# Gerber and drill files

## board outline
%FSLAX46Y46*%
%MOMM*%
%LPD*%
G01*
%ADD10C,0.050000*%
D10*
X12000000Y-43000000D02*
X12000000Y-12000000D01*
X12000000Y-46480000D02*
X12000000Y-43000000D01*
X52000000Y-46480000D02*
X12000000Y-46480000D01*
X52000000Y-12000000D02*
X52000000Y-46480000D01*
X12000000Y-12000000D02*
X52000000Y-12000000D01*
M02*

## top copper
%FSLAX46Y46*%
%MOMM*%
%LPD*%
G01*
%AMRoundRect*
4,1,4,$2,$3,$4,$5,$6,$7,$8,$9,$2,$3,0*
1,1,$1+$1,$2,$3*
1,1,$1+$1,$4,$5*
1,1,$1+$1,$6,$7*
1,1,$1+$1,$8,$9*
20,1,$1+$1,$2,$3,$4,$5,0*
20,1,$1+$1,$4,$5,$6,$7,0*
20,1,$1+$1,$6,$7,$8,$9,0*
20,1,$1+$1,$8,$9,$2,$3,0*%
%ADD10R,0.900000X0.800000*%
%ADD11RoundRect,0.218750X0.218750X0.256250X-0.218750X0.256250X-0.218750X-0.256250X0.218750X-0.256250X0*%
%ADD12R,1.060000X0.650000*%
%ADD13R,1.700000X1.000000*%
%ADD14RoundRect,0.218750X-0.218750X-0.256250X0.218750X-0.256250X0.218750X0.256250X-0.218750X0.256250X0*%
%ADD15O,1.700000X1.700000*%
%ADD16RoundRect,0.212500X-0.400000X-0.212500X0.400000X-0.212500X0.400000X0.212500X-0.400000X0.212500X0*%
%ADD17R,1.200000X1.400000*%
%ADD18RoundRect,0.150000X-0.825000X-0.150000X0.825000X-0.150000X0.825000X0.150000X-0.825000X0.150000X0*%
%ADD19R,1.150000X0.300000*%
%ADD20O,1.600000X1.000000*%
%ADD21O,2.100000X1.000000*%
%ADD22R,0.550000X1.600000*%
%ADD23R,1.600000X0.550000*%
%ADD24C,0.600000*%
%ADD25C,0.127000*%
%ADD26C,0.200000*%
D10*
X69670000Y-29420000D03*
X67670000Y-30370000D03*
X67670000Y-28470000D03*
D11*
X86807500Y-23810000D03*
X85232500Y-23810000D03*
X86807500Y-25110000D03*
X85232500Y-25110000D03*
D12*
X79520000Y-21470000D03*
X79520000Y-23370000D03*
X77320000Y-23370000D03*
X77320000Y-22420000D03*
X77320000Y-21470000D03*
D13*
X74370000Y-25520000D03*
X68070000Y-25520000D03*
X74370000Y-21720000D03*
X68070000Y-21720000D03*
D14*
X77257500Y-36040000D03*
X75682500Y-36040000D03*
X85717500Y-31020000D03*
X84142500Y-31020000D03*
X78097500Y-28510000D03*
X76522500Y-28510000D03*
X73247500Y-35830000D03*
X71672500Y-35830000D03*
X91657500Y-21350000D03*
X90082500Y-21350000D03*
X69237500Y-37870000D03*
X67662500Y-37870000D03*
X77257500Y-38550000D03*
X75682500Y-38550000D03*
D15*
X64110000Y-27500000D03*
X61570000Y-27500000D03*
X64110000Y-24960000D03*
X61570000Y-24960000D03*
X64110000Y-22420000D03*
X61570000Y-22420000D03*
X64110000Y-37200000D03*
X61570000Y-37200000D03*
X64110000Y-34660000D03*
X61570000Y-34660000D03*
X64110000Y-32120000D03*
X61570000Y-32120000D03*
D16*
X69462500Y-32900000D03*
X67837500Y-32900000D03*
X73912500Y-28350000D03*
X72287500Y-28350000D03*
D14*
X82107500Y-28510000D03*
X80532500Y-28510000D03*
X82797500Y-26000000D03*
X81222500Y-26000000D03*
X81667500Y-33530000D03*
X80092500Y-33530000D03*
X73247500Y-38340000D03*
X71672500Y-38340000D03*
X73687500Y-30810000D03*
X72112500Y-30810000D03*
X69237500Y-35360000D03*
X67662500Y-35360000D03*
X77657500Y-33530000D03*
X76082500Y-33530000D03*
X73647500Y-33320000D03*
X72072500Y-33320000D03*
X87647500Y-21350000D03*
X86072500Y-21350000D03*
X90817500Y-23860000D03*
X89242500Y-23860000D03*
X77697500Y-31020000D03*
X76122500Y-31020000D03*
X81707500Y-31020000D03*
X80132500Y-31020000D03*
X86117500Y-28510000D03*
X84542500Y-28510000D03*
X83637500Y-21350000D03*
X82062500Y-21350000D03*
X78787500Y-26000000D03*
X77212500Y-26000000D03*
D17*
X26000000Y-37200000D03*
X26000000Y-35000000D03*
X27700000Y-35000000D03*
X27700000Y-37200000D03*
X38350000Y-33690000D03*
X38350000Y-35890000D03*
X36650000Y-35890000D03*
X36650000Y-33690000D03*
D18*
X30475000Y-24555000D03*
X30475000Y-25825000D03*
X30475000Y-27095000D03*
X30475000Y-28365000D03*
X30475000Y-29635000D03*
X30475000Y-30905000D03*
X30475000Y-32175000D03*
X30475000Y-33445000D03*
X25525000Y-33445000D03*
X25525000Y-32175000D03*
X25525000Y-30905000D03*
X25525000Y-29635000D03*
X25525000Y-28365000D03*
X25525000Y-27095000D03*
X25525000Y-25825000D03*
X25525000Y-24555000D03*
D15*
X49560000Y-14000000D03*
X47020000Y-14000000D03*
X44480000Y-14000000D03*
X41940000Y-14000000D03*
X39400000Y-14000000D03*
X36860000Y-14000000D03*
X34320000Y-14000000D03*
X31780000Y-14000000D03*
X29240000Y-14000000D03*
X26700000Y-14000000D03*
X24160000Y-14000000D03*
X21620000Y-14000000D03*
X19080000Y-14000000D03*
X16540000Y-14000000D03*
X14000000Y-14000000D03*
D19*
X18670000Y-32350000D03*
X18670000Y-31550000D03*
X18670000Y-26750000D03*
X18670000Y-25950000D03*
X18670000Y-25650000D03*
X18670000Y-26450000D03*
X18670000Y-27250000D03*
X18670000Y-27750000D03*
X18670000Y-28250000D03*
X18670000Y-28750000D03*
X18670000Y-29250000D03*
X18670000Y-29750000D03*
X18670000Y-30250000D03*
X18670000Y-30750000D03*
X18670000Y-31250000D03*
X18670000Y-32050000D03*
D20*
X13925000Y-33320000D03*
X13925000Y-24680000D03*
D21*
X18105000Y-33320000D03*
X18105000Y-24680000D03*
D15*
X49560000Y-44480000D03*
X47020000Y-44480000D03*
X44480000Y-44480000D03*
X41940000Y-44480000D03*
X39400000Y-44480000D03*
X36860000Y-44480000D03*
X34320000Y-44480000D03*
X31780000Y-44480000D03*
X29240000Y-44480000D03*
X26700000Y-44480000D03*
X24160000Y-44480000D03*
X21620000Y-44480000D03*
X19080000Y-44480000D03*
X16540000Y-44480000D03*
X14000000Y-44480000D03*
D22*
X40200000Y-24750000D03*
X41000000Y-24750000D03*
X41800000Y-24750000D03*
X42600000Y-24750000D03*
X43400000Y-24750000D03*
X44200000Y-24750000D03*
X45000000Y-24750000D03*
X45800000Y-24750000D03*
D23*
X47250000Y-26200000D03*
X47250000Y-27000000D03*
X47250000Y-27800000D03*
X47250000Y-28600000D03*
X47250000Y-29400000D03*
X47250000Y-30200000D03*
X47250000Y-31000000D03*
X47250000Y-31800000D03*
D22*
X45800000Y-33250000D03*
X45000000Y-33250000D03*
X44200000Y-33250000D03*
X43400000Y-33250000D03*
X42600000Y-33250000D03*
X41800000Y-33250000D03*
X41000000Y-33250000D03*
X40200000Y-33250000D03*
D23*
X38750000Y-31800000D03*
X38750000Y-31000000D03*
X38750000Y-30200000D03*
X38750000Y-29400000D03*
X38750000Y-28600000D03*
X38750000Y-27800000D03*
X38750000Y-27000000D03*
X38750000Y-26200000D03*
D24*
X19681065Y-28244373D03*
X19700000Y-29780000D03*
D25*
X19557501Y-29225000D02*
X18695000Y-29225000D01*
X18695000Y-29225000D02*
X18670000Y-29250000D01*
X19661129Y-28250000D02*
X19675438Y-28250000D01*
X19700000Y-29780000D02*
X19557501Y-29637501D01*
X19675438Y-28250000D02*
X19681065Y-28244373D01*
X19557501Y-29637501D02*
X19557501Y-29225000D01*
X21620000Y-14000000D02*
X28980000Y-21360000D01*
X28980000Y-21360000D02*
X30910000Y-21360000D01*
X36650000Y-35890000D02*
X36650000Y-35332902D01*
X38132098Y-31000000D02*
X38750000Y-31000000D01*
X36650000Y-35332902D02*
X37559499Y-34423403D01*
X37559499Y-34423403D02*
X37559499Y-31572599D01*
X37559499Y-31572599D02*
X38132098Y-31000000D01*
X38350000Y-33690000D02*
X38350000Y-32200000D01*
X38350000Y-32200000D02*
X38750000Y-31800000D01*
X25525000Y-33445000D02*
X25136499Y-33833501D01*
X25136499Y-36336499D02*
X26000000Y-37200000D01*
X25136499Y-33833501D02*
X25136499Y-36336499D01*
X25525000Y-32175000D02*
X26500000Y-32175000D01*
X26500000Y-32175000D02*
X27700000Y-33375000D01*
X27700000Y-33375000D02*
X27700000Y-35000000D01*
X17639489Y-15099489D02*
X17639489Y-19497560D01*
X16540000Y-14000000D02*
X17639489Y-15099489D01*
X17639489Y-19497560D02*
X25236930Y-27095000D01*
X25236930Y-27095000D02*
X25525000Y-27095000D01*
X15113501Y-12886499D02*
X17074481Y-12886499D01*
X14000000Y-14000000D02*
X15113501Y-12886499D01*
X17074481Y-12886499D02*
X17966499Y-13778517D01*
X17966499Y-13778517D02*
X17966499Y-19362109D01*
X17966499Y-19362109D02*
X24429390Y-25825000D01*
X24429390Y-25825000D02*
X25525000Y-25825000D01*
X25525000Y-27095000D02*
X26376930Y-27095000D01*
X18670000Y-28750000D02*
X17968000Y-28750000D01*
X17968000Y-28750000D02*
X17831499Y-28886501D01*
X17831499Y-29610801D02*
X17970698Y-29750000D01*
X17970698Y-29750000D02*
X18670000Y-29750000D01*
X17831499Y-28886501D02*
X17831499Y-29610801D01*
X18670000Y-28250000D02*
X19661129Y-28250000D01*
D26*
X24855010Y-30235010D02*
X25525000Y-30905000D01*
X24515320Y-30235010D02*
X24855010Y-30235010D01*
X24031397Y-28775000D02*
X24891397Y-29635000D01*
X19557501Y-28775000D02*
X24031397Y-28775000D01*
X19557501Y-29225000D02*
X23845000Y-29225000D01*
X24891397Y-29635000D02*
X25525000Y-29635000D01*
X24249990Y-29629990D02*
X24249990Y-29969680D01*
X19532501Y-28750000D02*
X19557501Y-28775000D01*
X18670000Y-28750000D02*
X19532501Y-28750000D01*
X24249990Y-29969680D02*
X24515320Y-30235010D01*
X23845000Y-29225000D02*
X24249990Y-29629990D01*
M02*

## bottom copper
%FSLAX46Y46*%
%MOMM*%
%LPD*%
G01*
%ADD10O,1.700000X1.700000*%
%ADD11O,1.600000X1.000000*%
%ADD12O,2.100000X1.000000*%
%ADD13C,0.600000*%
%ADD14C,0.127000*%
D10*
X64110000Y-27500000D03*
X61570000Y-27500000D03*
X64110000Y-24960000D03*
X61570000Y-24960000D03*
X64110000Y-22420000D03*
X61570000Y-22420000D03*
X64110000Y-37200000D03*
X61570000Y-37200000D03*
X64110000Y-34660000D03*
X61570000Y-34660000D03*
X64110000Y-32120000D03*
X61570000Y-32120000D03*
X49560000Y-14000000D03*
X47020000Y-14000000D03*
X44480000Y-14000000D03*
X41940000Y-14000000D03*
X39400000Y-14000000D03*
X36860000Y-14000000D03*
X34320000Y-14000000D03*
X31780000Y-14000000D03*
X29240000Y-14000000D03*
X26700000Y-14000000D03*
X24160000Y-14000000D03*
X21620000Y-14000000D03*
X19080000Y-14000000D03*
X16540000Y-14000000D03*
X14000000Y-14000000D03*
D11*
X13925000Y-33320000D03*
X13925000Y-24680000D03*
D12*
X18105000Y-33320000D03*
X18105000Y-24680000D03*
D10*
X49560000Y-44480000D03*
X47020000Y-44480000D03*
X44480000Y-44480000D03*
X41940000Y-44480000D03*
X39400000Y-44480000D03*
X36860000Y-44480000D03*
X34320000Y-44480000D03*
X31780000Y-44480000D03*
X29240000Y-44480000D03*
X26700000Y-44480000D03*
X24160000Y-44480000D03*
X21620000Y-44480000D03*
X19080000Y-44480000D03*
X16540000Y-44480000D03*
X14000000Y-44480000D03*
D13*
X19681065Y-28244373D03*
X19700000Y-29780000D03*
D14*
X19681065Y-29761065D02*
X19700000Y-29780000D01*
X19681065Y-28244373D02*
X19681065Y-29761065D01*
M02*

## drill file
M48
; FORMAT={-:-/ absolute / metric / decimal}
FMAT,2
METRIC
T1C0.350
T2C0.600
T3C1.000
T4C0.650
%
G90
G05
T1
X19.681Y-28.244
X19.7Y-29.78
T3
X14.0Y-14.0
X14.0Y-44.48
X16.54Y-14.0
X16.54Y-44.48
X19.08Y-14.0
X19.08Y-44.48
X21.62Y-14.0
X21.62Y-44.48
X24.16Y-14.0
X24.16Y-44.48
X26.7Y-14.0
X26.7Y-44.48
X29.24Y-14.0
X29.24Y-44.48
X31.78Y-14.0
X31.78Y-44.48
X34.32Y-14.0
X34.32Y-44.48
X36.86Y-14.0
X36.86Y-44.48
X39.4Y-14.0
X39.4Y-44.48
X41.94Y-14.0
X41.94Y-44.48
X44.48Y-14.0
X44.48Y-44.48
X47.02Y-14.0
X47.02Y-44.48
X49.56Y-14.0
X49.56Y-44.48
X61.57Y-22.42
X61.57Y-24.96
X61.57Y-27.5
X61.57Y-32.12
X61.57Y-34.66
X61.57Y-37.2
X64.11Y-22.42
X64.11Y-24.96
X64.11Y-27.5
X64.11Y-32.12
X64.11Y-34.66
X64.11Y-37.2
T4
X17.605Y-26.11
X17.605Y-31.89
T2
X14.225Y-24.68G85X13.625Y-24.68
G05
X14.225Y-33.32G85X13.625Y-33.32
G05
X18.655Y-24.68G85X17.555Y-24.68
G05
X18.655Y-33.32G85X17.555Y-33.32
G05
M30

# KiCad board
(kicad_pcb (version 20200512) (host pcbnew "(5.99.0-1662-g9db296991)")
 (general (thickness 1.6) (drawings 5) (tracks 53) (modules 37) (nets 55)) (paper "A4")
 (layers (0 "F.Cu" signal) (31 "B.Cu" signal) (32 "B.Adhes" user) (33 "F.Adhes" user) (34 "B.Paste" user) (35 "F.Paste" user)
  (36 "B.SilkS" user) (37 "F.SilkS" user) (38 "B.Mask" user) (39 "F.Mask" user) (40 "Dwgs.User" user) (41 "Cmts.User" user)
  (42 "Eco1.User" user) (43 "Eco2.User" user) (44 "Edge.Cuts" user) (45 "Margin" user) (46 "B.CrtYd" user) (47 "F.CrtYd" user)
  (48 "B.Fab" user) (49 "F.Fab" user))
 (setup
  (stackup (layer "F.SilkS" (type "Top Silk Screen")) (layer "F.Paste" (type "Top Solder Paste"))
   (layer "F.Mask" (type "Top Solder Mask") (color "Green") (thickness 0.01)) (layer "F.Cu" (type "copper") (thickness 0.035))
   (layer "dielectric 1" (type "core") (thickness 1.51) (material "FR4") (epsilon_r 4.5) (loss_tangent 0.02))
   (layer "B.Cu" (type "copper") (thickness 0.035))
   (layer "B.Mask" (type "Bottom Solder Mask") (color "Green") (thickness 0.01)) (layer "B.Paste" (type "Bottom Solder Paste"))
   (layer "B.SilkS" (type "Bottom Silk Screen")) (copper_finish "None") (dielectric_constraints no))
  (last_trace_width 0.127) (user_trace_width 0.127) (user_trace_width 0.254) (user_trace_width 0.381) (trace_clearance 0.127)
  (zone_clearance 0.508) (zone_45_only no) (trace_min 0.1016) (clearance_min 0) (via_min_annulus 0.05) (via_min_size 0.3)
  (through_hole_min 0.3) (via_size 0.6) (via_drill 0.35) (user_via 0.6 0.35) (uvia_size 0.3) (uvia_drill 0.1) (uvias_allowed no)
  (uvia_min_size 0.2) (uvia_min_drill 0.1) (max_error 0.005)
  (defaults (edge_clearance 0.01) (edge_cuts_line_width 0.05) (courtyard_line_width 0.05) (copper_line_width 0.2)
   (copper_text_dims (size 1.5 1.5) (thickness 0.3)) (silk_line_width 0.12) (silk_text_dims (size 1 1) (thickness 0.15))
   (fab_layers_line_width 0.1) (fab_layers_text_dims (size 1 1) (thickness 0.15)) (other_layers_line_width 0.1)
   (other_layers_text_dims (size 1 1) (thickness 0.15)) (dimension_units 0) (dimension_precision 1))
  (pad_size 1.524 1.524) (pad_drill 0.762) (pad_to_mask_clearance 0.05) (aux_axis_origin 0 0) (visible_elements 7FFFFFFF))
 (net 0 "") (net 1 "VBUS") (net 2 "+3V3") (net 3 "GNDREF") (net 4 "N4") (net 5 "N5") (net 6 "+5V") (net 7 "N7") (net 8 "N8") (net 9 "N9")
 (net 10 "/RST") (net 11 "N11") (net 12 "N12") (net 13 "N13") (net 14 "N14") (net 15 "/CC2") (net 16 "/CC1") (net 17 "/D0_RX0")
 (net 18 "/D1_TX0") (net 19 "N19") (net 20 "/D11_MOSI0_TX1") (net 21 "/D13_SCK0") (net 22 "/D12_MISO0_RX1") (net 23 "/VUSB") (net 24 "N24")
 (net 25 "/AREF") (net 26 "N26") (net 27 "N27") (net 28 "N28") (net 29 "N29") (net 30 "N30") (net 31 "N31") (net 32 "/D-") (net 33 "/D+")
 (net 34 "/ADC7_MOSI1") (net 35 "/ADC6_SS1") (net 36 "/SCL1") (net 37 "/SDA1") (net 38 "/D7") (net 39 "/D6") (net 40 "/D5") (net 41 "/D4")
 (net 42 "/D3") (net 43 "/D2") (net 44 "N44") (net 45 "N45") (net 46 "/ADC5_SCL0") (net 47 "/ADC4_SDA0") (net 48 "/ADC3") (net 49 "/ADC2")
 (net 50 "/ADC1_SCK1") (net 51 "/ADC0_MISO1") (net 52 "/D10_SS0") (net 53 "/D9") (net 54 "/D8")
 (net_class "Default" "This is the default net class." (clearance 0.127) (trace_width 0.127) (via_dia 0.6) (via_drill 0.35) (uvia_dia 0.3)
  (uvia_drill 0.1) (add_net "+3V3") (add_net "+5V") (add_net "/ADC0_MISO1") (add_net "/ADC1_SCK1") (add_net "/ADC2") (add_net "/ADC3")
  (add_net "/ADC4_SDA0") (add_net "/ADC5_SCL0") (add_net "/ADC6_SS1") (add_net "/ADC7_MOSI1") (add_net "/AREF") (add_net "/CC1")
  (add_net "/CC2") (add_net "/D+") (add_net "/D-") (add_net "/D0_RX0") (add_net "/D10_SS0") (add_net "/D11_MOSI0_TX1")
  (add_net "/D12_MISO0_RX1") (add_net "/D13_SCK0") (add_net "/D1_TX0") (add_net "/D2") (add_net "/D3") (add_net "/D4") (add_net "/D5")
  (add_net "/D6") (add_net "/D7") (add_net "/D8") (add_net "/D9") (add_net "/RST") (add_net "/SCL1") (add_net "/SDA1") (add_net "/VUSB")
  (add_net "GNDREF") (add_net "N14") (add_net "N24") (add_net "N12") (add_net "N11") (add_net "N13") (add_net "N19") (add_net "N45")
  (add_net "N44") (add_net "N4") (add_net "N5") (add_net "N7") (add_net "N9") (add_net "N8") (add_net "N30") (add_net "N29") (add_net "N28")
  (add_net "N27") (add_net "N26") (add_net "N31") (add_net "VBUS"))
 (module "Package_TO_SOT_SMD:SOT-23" (layer "F.Cu") (at 68.67 29.42)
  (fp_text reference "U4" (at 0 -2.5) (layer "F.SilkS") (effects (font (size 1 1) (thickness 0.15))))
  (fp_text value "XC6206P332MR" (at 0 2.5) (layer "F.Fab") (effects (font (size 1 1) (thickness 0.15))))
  (pad "3" smd rect (at 1 0) (size 0.9 0.8) (layers "F.Cu" "F.Paste" "F.Mask") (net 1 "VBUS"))
  (pad "2" smd rect (at -1 0.95) (size 0.9 0.8) (layers "F.Cu" "F.Paste" "F.Mask") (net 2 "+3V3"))
  (pad "1" smd rect (at -1 -0.95) (size 0.9 0.8) (layers "F.Cu" "F.Paste" "F.Mask") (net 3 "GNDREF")))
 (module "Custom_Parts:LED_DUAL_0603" (layer "F.Cu") (at 86.02 24.46)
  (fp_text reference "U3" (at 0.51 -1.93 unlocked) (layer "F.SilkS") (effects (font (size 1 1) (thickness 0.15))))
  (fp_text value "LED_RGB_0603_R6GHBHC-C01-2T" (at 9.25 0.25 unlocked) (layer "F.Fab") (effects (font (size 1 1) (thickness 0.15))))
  (pad "2" smd roundrect (at 0.7875 -0.65 180) (size 0.875 0.95) (layers "F.Cu" "F.Paste" "F.Mask") (roundrect_rratio 0.25) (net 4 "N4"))
  (pad "3" smd roundrect (at -0.7875 -0.65 180) (size 0.875 0.95) (layers "F.Cu" "F.Paste" "F.Mask") (roundrect_rratio 0.25) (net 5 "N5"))
  (pad "1" smd roundrect (at 0.7875 0.65 180) (size 0.875 0.95) (layers "F.Cu" "F.Paste" "F.Mask") (roundrect_rratio 0.25) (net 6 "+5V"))
  (pad "4" smd roundrect (at -0.7875 0.65 180) (size 0.875 0.95) (layers "F.Cu" "F.Paste" "F.Mask") (roundrect_rratio 0.25) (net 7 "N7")))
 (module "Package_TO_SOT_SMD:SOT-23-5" (layer "F.Cu") (at 78.42 22.42)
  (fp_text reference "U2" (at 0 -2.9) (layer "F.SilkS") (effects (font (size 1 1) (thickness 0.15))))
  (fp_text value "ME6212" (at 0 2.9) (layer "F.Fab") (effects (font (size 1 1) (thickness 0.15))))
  (pad "5" smd rect (at 1.1 -0.95) (size 1.06 0.65) (layers "F.Cu" "F.Paste" "F.Mask") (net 6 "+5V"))
  (pad "4" smd rect (at 1.1 0.95) (size 1.06 0.65) (layers "F.Cu" "F.Paste" "F.Mask") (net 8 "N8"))
  (pad "3" smd rect (at -1.1 0.95) (size 1.06 0.65) (layers "F.Cu" "F.Paste" "F.Mask") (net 1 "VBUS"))
  (pad "2" smd rect (at -1.1 0) (size 1.06 0.65) (layers "F.Cu" "F.Paste" "F.Mask") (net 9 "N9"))
  (pad "1" smd rect (at -1.1 -0.95) (size 1.06 0.65) (layers "F.Cu" "F.Paste" "F.Mask") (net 1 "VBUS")))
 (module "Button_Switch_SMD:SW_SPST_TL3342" (layer "F.Cu") (at 71.22 23.62)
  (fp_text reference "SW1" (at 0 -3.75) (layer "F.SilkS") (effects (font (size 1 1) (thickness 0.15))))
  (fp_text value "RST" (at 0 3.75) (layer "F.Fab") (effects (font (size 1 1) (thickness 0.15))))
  (pad "2" smd rect (at 3.15 1.9) (size 1.7 1) (layers "F.Cu" "F.Paste" "F.Mask") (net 3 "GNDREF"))
  (pad "2" smd rect (at -3.15 1.9) (size 1.7 1) (layers "F.Cu" "F.Paste" "F.Mask") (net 3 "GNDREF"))
  (pad "1" smd rect (at 3.15 -1.9) (size 1.7 1) (layers "F.Cu" "F.Paste" "F.Mask") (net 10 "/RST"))
  (pad "1" smd rect (at -3.15 -1.9) (size 1.7 1) (layers "F.Cu" "F.Paste" "F.Mask") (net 10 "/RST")))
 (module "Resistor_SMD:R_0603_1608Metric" (layer "F.Cu") (at 76.47 36.04)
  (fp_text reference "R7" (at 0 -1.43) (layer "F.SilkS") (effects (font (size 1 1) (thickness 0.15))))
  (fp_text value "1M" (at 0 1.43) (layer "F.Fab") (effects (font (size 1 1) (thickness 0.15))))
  (pad "2" smd roundrect (at 0.7875 0) (size 0.875 0.95) (layers "F.Cu" "F.Paste" "F.Mask") (roundrect_rratio 0.25) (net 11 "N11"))
  (pad "1" smd roundrect (at -0.7875 0) (size 0.875 0.95) (layers "F.Cu" "F.Paste" "F.Mask") (roundrect_rratio 0.25) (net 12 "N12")))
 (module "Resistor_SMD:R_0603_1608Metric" (layer "F.Cu") (at 84.93 31.02)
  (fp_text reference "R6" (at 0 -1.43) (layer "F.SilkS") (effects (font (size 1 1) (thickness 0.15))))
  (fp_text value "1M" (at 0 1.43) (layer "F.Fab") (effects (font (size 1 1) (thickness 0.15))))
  (pad "2" smd roundrect (at 0.7875 0) (size 0.875 0.95) (layers "F.Cu" "F.Paste" "F.Mask") (roundrect_rratio 0.25) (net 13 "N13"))
  (pad "1" smd roundrect (at -0.7875 0) (size 0.875 0.95) (layers "F.Cu" "F.Paste" "F.Mask") (roundrect_rratio 0.25) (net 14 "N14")))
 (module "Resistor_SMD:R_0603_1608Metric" (layer "F.Cu") (at 77.31 28.51)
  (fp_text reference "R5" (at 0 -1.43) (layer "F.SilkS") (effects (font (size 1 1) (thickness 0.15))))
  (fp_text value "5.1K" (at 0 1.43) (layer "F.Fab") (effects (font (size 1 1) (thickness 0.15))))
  (pad "2" smd roundrect (at 0.7875 0) (size 0.875 0.95) (layers "F.Cu" "F.Paste" "F.Mask") (roundrect_rratio 0.25) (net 3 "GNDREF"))
  (pad "1" smd roundrect (at -0.7875 0) (size 0.875 0.95) (layers "F.Cu" "F.Paste" "F.Mask") (roundrect_rratio 0.25) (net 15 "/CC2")))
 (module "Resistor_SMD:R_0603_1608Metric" (layer "F.Cu") (at 72.46 35.83)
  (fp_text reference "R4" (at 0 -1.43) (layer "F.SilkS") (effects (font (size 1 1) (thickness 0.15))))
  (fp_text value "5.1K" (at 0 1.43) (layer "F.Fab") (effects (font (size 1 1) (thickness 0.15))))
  (pad "2" smd roundrect (at 0.7875 0) (size 0.875 0.95) (layers "F.Cu" "F.Paste" "F.Mask") (roundrect_rratio 0.25) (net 3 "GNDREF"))
  (pad "1" smd roundrect (at -0.7875 0) (size 0.875 0.95) (layers "F.Cu" "F.Paste" "F.Mask") (roundrect_rratio 0.25) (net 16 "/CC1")))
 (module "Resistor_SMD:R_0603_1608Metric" (layer "F.Cu") (at 90.87 21.35)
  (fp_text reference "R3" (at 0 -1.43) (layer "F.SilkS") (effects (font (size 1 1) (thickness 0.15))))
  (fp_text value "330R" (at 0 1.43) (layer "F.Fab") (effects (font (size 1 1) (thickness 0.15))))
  (pad "2" smd roundrect (at 0.7875 0) (size 0.875 0.95) (layers "F.Cu" "F.Paste" "F.Mask") (roundrect_rratio 0.25) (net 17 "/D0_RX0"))
  (pad "1" smd roundrect (at -0.7875 0) (size 0.875 0.95) (layers "F.Cu" "F.Paste" "F.Mask") (roundrect_rratio 0.25) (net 7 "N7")))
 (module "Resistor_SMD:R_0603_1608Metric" (layer "F.Cu") (at 68.45 37.87)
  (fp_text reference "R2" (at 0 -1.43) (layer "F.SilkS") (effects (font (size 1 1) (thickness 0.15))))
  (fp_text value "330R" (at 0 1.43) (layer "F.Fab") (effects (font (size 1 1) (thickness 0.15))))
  (pad "2" smd roundrect (at 0.7875 0) (size 0.875 0.95) (layers "F.Cu" "F.Paste" "F.Mask") (roundrect_rratio 0.25) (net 3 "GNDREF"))
  (pad "1" smd roundrect (at -0.7875 0) (size 0.875 0.95) (layers "F.Cu" "F.Paste" "F.Mask") (roundrect_rratio 0.25) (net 5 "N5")))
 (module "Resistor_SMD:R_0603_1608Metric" (layer "F.Cu") (at 76.47 38.55)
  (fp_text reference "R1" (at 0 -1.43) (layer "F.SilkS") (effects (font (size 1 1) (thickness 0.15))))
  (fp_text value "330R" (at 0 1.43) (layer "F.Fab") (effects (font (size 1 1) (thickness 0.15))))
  (pad "2" smd roundrect (at 0.7875 0) (size 0.875 0.95) (layers "F.Cu" "F.Paste" "F.Mask") (roundrect_rratio 0.25) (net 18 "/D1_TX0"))
  (pad "1" smd roundrect (at -0.7875 0) (size 0.875 0.95) (layers "F.Cu" "F.Paste" "F.Mask") (roundrect_rratio 0.25) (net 4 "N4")))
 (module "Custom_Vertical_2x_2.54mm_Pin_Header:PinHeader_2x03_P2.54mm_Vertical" (layer "F.Cu") (at 61.57 22.42)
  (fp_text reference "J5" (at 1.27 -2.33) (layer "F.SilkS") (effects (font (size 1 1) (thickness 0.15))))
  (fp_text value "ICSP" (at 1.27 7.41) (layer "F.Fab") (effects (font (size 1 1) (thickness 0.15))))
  (pad "6" thru_hole oval (at 2.54 5.08) (size 1.7 1.7) (drill 1) (layers *.Cu *.Mask) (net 3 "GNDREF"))
  (pad "5" thru_hole oval (at 0 5.08) (size 1.7 1.7) (drill 1) (layers *.Cu *.Mask) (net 3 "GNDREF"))
  (pad "4" thru_hole oval (at 2.54 2.54) (size 1.7 1.7) (drill 1) (layers *.Cu *.Mask) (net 6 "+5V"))
  (pad "3" thru_hole oval (at 0 2.54) (size 1.7 1.7) (drill 1) (layers *.Cu *.Mask) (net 2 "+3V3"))
  (pad "2" thru_hole oval (at 2.54 0) (size 1.7 1.7) (drill 1) (layers *.Cu *.Mask) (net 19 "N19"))
  (pad "1" thru_hole oval (at 0 0) (size 1.7 1.7) (drill 1) (layers *.Cu *.Mask) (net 6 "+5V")))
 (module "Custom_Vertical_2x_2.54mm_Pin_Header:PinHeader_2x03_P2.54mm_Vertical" (layer "F.Cu") (at 61.57 32.12)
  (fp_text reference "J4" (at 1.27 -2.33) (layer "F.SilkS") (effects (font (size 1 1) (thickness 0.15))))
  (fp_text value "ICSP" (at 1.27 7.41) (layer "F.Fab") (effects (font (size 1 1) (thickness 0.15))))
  (pad "6" thru_hole oval (at 2.54 5.08) (size 1.7 1.7) (drill 1) (layers *.Cu *.Mask) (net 3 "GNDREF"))
  (pad "5" thru_hole oval (at 0 5.08) (size 1.7 1.7) (drill 1) (layers *.Cu *.Mask) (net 10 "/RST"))
  (pad "4" thru_hole oval (at 2.54 2.54) (size 1.7 1.7) (drill 1) (layers *.Cu *.Mask) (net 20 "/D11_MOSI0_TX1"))
  (pad "3" thru_hole oval (at 0 2.54) (size 1.7 1.7) (drill 1) (layers *.Cu *.Mask) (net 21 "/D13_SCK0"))
  (pad "2" thru_hole oval (at 2.54 0) (size 1.7 1.7) (drill 1) (layers *.Cu *.Mask) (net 6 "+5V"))
  (pad "1" thru_hole oval (at 0 0) (size 1.7 1.7) (drill 1) (layers *.Cu *.Mask) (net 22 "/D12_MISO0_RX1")))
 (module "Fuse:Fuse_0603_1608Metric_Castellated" (layer "F.Cu") (at 68.65 32.9)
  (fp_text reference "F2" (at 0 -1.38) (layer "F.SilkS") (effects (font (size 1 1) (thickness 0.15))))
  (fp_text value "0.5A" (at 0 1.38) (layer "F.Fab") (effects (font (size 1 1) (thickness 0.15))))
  (pad "2" smd roundrect (at 0.8125 0) (size 1.225 0.85) (layers "F.Cu" "F.Paste" "F.Mask") (roundrect_rratio 0.25) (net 1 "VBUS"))
  (pad "1" smd roundrect (at -0.8125 0) (size 1.225 0.85) (layers "F.Cu" "F.Paste" "F.Mask") (roundrect_rratio 0.25) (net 19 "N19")))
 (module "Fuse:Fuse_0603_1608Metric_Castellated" (layer "F.Cu") (at 73.1 28.35)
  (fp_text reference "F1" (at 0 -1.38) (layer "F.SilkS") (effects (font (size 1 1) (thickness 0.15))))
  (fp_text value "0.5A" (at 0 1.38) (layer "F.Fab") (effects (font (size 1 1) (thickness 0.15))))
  (pad "2" smd roundrect (at 0.8125 0) (size 1.225 0.85) (layers "F.Cu" "F.Paste" "F.Mask") (roundrect_rratio 0.25) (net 1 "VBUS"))
  (pad "1" smd roundrect (at -0.8125 0) (size 1.225 0.85) (layers "F.Cu" "F.Paste" "F.Mask") (roundrect_rratio 0.25) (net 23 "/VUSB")))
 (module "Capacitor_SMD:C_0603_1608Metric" (layer "F.Cu") (at 81.32 28.51)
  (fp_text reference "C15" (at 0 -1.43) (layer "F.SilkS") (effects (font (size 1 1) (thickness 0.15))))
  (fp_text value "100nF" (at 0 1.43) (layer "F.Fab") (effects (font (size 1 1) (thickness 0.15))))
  (pad "2" smd roundrect (at 0.7875 0) (size 0.875 0.95) (layers "F.Cu" "F.Paste" "F.Mask") (roundrect_rratio 0.25) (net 3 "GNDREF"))
  (pad "1" smd roundrect (at -0.7875 0) (size 0.875 0.95) (layers "F.Cu" "F.Paste" "F.Mask") (roundrect_rratio 0.25) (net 6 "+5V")))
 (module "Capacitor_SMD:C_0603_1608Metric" (layer "F.Cu") (at 82.01 26)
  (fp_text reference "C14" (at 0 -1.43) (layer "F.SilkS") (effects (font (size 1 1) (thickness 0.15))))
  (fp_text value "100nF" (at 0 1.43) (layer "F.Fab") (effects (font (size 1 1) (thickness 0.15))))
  (pad "2" smd roundrect (at 0.7875 0) (size 0.875 0.95) (layers "F.Cu" "F.Paste" "F.Mask") (roundrect_rratio 0.25) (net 3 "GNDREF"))
  (pad "1" smd roundrect (at -0.7875 0) (size 0.875 0.95) (layers "F.Cu" "F.Paste" "F.Mask") (roundrect_rratio 0.25) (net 6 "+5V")))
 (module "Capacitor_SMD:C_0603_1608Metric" (layer "F.Cu") (at 80.88 33.53)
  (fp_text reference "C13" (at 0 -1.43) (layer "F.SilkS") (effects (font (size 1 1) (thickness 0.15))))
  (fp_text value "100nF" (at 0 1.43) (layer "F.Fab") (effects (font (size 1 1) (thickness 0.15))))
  (pad "2" smd roundrect (at 0.7875 0) (size 0.875 0.95) (layers "F.Cu" "F.Paste" "F.Mask") (roundrect_rratio 0.25) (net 3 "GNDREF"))
  (pad "1" smd roundrect (at -0.7875 0) (size 0.875 0.95) (layers "F.Cu" "F.Paste" "F.Mask") (roundrect_rratio 0.25) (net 11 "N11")))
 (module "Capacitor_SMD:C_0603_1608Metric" (layer "F.Cu") (at 72.46 38.34)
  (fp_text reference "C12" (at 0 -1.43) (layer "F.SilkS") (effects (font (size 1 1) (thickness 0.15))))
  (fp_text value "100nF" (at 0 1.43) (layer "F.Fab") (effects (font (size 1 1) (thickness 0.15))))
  (pad "2" smd roundrect (at 0.7875 0) (size 0.875 0.95) (layers "F.Cu" "F.Paste" "F.Mask") (roundrect_rratio 0.25) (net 3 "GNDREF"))
  (pad "1" smd roundrect (at -0.7875 0) (size 0.875 0.95) (layers "F.Cu" "F.Paste" "F.Mask") (roundrect_rratio 0.25) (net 12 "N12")))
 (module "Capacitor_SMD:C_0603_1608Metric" (layer "F.Cu") (at 72.9 30.81)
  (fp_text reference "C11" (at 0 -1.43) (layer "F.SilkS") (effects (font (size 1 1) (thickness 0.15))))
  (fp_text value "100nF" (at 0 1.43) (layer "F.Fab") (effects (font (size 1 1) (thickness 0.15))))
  (pad "2" smd roundrect (at 0.7875 0) (size 0.875 0.95) (layers "F.Cu" "F.Paste" "F.Mask") (roundrect_rratio 0.25) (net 10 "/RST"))
  (pad "1" smd roundrect (at -0.7875 0) (size 0.875 0.95) (layers "F.Cu" "F.Paste" "F.Mask") (roundrect_rratio 0.25) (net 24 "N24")))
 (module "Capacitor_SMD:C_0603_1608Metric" (layer "F.Cu") (at 68.45 35.36)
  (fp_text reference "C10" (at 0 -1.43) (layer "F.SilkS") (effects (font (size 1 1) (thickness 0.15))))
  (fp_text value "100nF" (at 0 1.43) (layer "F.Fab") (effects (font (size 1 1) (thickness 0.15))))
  (pad "2" smd roundrect (at 0.7875 0) (size 0.875 0.95) (layers "F.Cu" "F.Paste" "F.Mask") (roundrect_rratio 0.25) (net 3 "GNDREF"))
  (pad "1" smd roundrect (at -0.7875 0) (size 0.875 0.95) (layers "F.Cu" "F.Paste" "F.Mask") (roundrect_rratio 0.25) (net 14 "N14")))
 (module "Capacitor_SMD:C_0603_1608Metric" (layer "F.Cu") (at 76.87 33.53)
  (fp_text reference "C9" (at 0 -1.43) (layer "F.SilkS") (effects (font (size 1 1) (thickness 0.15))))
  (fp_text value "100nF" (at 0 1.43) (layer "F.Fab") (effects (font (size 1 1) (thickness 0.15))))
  (pad "2" smd roundrect (at 0.7875 0) (size 0.875 0.95) (layers "F.Cu" "F.Paste" "F.Mask") (roundrect_rratio 0.25) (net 3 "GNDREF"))
  (pad "1" smd roundrect (at -0.7875 0) (size 0.875 0.95) (layers "F.Cu" "F.Paste" "F.Mask") (roundrect_rratio 0.25) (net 13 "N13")))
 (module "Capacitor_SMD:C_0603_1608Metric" (layer "F.Cu") (at 72.86 33.32)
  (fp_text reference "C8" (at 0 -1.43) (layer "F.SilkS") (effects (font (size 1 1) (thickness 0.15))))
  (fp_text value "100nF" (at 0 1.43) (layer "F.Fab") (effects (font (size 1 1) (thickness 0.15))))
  (pad "2" smd roundrect (at 0.7875 0) (size 0.875 0.95) (layers "F.Cu" "F.Paste" "F.Mask") (roundrect_rratio 0.25) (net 3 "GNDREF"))
  (pad "1" smd roundrect (at -0.7875 0) (size 0.875 0.95) (layers "F.Cu" "F.Paste" "F.Mask") (roundrect_rratio 0.25) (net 1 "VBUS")))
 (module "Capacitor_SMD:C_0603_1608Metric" (layer "F.Cu") (at 86.86 21.35)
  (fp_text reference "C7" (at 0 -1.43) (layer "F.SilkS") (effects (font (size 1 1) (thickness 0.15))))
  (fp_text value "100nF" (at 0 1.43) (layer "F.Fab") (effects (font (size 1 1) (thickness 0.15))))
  (pad "2" smd roundrect (at 0.7875 0) (size 0.875 0.95) (layers "F.Cu" "F.Paste" "F.Mask") (roundrect_rratio 0.25) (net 3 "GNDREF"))
  (pad "1" smd roundrect (at -0.7875 0) (size 0.875 0.95) (layers "F.Cu" "F.Paste" "F.Mask") (roundrect_rratio 0.25) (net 6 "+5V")))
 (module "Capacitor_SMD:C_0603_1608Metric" (layer "F.Cu") (at 90.03 23.86)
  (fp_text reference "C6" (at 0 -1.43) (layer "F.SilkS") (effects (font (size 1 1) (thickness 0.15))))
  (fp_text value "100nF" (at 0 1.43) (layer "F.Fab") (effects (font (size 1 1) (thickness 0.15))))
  (pad "2" smd roundrect (at 0.7875 0) (size 0.875 0.95) (layers "F.Cu" "F.Paste" "F.Mask") (roundrect_rratio 0.25) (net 3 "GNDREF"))
  (pad "1" smd roundrect (at -0.7875 0) (size 0.875 0.95) (layers "F.Cu" "F.Paste" "F.Mask") (roundrect_rratio 0.25) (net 2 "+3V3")))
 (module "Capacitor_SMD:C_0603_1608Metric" (layer "F.Cu") (at 76.91 31.02)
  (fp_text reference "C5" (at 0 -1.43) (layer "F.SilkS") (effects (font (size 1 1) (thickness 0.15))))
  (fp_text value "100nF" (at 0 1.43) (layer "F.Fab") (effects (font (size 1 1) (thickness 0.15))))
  (pad "2" smd roundrect (at 0.7875 0) (size 0.875 0.95) (layers "F.Cu" "F.Paste" "F.Mask") (roundrect_rratio 0.25) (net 3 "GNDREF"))
  (pad "1" smd roundrect (at -0.7875 0) (size 0.875 0.95) (layers "F.Cu" "F.Paste" "F.Mask") (roundrect_rratio 0.25) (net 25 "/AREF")))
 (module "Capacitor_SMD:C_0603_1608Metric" (layer "F.Cu") (at 80.92 31.02)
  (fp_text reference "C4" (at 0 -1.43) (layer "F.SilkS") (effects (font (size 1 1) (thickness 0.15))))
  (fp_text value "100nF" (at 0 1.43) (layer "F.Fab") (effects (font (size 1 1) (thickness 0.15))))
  (pad "2" smd roundrect (at 0.7875 0) (size 0.875 0.95) (layers "F.Cu" "F.Paste" "F.Mask") (roundrect_rratio 0.25) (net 3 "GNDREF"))
  (pad "1" smd roundrect (at -0.7875 0) (size 0.875 0.95) (layers "F.Cu" "F.Paste" "F.Mask") (roundrect_rratio 0.25) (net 2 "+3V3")))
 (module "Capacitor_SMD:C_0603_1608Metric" (layer "F.Cu") (at 85.33 28.51)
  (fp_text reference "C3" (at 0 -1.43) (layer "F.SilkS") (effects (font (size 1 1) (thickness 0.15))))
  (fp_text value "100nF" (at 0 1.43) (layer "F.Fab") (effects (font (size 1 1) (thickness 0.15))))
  (pad "2" smd roundrect (at 0.7875 0) (size 0.875 0.95) (layers "F.Cu" "F.Paste" "F.Mask") (roundrect_rratio 0.25) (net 3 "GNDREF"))
  (pad "1" smd roundrect (at -0.7875 0) (size 0.875 0.95) (layers "F.Cu" "F.Paste" "F.Mask") (roundrect_rratio 0.25) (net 1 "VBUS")))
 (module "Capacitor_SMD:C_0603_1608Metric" (layer "F.Cu") (at 82.85 21.35)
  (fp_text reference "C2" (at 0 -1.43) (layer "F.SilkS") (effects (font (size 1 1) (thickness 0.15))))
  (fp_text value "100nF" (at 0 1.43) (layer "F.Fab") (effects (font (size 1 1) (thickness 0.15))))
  (pad "2" smd roundrect (at 0.7875 0) (size 0.875 0.95) (layers "F.Cu" "F.Paste" "F.Mask") (roundrect_rratio 0.25) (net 3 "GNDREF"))
  (pad "1" smd roundrect (at -0.7875 0) (size 0.875 0.95) (layers "F.Cu" "F.Paste" "F.Mask") (roundrect_rratio 0.25) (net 6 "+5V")))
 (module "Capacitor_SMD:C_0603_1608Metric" (layer "F.Cu") (at 78 26)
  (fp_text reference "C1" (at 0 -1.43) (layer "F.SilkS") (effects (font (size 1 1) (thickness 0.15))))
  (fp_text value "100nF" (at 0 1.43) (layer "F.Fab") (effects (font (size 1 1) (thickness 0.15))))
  (pad "2" smd roundrect (at 0.7875 0) (size 0.875 0.95) (layers "F.Cu" "F.Paste" "F.Mask") (roundrect_rratio 0.25) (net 3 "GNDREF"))
  (pad "1" smd roundrect (at -0.7875 0) (size 0.875 0.95) (layers "F.Cu" "F.Paste" "F.Mask") (roundrect_rratio 0.25) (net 1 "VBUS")))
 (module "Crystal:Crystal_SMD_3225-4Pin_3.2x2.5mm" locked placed (layer "F.Cu") (at 26.85 36.1 90)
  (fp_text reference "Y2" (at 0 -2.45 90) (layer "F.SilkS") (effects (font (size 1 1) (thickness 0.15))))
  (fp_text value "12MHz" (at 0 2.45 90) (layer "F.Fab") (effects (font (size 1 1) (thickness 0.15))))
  (pad "4" smd rect (at -1.1 -0.85 90) (size 1.4 1.2) (layers "F.Cu" "F.Paste" "F.Mask") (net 11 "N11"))
  (pad "3" smd rect (at 1.1 -0.85 90) (size 1.4 1.2) (layers "F.Cu" "F.Paste" "F.Mask") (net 3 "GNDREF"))
  (pad "2" smd rect (at 1.1 0.85 90) (size 1.4 1.2) (layers "F.Cu" "F.Paste" "F.Mask") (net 12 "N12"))
  (pad "1" smd rect (at -1.1 0.85 90) (size 1.4 1.2) (layers "F.Cu" "F.Paste" "F.Mask") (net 3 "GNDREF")))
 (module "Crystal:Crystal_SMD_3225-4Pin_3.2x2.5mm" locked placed (layer "F.Cu") (at 37.5 34.79 -90)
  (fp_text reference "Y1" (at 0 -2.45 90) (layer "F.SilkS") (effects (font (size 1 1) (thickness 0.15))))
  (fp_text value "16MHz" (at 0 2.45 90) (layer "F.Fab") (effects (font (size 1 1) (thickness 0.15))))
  (pad "4" smd rect (at -1.1 -0.85 270) (size 1.4 1.2) (layers "F.Cu" "F.Paste" "F.Mask") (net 13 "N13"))
  (pad "3" smd rect (at 1.1 -0.85 270) (size 1.4 1.2) (layers "F.Cu" "F.Paste" "F.Mask") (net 3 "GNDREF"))
  (pad "2" smd rect (at 1.1 0.85 270) (size 1.4 1.2) (layers "F.Cu" "F.Paste" "F.Mask") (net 14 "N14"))
  (pad "1" smd rect (at -1.1 0.85 270) (size 1.4 1.2) (layers "F.Cu" "F.Paste" "F.Mask") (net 3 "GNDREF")))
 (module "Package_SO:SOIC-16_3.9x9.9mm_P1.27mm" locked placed (layer "F.Cu") (at 28 29)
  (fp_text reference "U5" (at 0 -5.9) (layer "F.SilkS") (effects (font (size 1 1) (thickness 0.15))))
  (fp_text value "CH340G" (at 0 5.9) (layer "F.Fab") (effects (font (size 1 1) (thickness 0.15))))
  (pad "16" smd roundrect (at 2.475 -4.445) (size 1.95 0.6) (layers "F.Cu" "F.Paste" "F.Mask") (roundrect_rratio 0.25) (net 6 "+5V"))
  (pad "15" smd roundrect (at 2.475 -3.175) (size 1.95 0.6) (layers "F.Cu" "F.Paste" "F.Mask") (roundrect_rratio 0.25) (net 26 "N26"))
  (pad "14" smd roundrect (at 2.475 -1.905) (size 1.95 0.6) (layers "F.Cu" "F.Paste" "F.Mask") (roundrect_rratio 0.25) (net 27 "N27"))
  (pad "13" smd roundrect (at 2.475 -0.635) (size 1.95 0.6) (layers "F.Cu" "F.Paste" "F.Mask") (roundrect_rratio 0.25) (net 24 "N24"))
  (pad "12" smd roundrect (at 2.475 0.635) (size 1.95 0.6) (layers "F.Cu" "F.Paste" "F.Mask") (roundrect_rratio 0.25) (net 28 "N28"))
  (pad "11" smd roundrect (at 2.475 1.905) (size 1.95 0.6) (layers "F.Cu" "F.Paste" "F.Mask") (roundrect_rratio 0.25) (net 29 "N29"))
  (pad "10" smd roundrect (at 2.475 3.175) (size 1.95 0.6) (layers "F.Cu" "F.Paste" "F.Mask") (roundrect_rratio 0.25) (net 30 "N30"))
  (pad "9" smd roundrect (at 2.475 4.445) (size 1.95 0.6) (layers "F.Cu" "F.Paste" "F.Mask") (roundrect_rratio 0.25) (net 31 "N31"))
  (pad "8" smd roundrect (at -2.475 4.445) (size 1.95 0.6) (layers "F.Cu" "F.Paste" "F.Mask") (roundrect_rratio 0.25) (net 11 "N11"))
  (pad "7" smd roundrect (at -2.475 3.175) (size 1.95 0.6) (layers "F.Cu" "F.Paste" "F.Mask") (roundrect_rratio 0.25) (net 12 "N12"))
  (pad "6" smd roundrect (at -2.475 1.905) (size 1.95 0.6) (layers "F.Cu" "F.Paste" "F.Mask") (roundrect_rratio 0.25) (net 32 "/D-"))
  (pad "5" smd roundrect (at -2.475 0.635) (size 1.95 0.6) (layers "F.Cu" "F.Paste" "F.Mask") (roundrect_rratio 0.25) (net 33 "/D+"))
  (pad "4" smd roundrect (at -2.475 -0.635) (size 1.95 0.6) (layers "F.Cu" "F.Paste" "F.Mask") (roundrect_rratio 0.25) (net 2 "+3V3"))
  (pad "3" smd roundrect (at -2.475 -1.905) (size 1.95 0.6) (layers "F.Cu" "F.Paste" "F.Mask") (roundrect_rratio 0.25) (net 18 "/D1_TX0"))
  (pad "2" smd roundrect (at -2.475 -3.175) (size 1.95 0.6) (layers "F.Cu" "F.Paste" "F.Mask") (roundrect_rratio 0.25) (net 17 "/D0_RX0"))
  (pad "1" smd roundrect (at -2.475 -4.445) (size 1.95 0.6) (layers "F.Cu" "F.Paste" "F.Mask") (roundrect_rratio 0.25) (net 3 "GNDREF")))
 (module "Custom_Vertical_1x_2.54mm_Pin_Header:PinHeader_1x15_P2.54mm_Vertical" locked (layer "F.Cu") (at 14 14 90)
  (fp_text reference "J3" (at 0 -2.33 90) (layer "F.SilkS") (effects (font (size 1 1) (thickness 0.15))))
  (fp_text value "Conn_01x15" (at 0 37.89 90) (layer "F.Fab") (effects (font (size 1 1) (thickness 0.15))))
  (pad "15" thru_hole oval (at 0 35.56 90) (size 1.7 1.7) (drill 1) (layers *.Cu *.Mask) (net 3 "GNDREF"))
  (pad "14" thru_hole oval (at 0 33.02 90) (size 1.7 1.7) (drill 1) (layers *.Cu *.Mask) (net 6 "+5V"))
  (pad "13" thru_hole oval (at 0 30.48 90) (size 1.7 1.7) (drill 1) (layers *.Cu *.Mask) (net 25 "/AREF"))
  (pad "12" thru_hole oval (at 0 27.94 90) (size 1.7 1.7) (drill 1) (layers *.Cu *.Mask) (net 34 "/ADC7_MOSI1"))
  (pad "11" thru_hole oval (at 0 25.4 90) (size 1.7 1.7) (drill 1) (layers *.Cu *.Mask) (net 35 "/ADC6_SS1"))
  (pad "10" thru_hole oval (at 0 22.86 90) (size 1.7 1.7) (drill 1) (layers *.Cu *.Mask) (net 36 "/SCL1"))
  (pad "9" thru_hole oval (at 0 20.32 90) (size 1.7 1.7) (drill 1) (layers *.Cu *.Mask) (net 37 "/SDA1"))
  (pad "8" thru_hole oval (at 0 17.78 90) (size 1.7 1.7) (drill 1) (layers *.Cu *.Mask) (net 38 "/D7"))
  (pad "7" thru_hole oval (at 0 15.24 90) (size 1.7 1.7) (drill 1) (layers *.Cu *.Mask) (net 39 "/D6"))
  (pad "6" thru_hole oval (at 0 12.7 90) (size 1.7 1.7) (drill 1) (layers *.Cu *.Mask) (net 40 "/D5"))
  (pad "5" thru_hole oval (at 0 10.16 90) (size 1.7 1.7) (drill 1) (layers *.Cu *.Mask) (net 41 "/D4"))
  (pad "4" thru_hole oval (at 0 7.62 90) (size 1.7 1.7) (drill 1) (layers *.Cu *.Mask) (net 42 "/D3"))
  (pad "3" thru_hole oval (at 0 5.08 90) (size 1.7 1.7) (drill 1) (layers *.Cu *.Mask) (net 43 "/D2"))
  (pad "2" thru_hole oval (at 0 2.54 90) (size 1.7 1.7) (drill 1) (layers *.Cu *.Mask) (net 18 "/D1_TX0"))
  (pad "1" thru_hole oval (at 0 0 90) (size 1.7 1.7) (drill 1) (layers *.Cu *.Mask) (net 17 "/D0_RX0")))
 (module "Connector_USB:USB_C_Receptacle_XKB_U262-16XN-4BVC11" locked (layer "F.Cu") (at 15 29 -90)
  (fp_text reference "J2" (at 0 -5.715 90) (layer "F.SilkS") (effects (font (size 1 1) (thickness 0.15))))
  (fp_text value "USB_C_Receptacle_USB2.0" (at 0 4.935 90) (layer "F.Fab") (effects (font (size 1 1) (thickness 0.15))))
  (pad "A12" smd rect (at 3.35 -3.67 270) (size 0.3 1.15) (layers "F.Cu" "F.Paste" "F.Mask") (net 3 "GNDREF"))
  (pad "A9" smd rect (at 2.55 -3.67 270) (size 0.3 1.15) (layers "F.Cu" "F.Paste" "F.Mask") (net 23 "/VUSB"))
  (pad "B9" smd rect (at -2.25 -3.67 270) (size 0.3 1.15) (layers "F.Cu" "F.Paste" "F.Mask") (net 23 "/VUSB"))
  (pad "B12" smd rect (at -3.05 -3.67 270) (size 0.3 1.15) (layers "F.Cu" "F.Paste" "F.Mask") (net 3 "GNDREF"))
  (pad "A1" smd rect (at -3.35 -3.67 270) (size 0.3 1.15) (layers "F.Cu" "F.Paste" "F.Mask") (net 3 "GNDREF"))
  (pad "A4" smd rect (at -2.55 -3.67 270) (size 0.3 1.15) (layers "F.Cu" "F.Paste" "F.Mask") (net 23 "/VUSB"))
  (pad "B8" smd rect (at -1.75 -3.67 270) (size 0.3 1.15) (layers "F.Cu" "F.Paste" "F.Mask") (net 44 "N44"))
  (pad "A5" smd rect (at -1.25 -3.67 270) (size 0.3 1.15) (layers "F.Cu" "F.Paste" "F.Mask") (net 16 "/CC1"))
  (pad "B7" smd rect (at -0.75 -3.67 270) (size 0.3 1.15) (layers "F.Cu" "F.Paste" "F.Mask") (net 32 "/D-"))
  (pad "A6" smd rect (at -0.25 -3.67 270) (size 0.3 1.15) (layers "F.Cu" "F.Paste" "F.Mask") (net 33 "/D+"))
  (pad "A7" smd rect (at 0.25 -3.67 270) (size 0.3 1.15) (layers "F.Cu" "F.Paste" "F.Mask") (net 32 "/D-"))
  (pad "B6" smd rect (at 0.75 -3.67 270) (size 0.3 1.15) (layers "F.Cu" "F.Paste" "F.Mask") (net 33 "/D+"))
  (pad "A8" smd rect (at 1.25 -3.67 270) (size 0.3 1.15) (layers "F.Cu" "F.Paste" "F.Mask") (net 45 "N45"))
  (pad "B5" smd rect (at 1.75 -3.67 270) (size 0.3 1.15) (layers "F.Cu" "F.Paste" "F.Mask") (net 15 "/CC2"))
  (pad "B4" smd rect (at 2.25 -3.67 270) (size 0.3 1.15) (layers "F.Cu" "F.Paste" "F.Mask") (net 23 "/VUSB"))
  (pad "B1" smd rect (at 3.05 -3.67 270) (size 0.3 1.15) (layers "F.Cu" "F.Paste" "F.Mask") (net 3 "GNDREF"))
  (pad "" np_thru_hole circle (at -2.89 -2.605 270) (size 0.65 0.65) (drill 0.65) (layers *.Cu *.Mask))
  (pad "" np_thru_hole circle (at 2.89 -2.605 270) (size 0.65 0.65) (drill 0.65) (layers *.Cu *.Mask))
  (pad "S1" thru_hole oval (at 4.32 1.075 270) (size 1 1.6) (drill oval 0.6 1.2) (layers *.Cu *.Mask) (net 3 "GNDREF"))
  (pad "S1" thru_hole oval (at -4.32 1.075 270) (size 1 1.6) (drill oval 0.6 1.2) (layers *.Cu *.Mask) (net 3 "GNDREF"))
  (pad "S1" thru_hole oval (at 4.32 -3.105 270) (size 1 2.1) (drill oval 0.6 1.7) (layers *.Cu *.Mask) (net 3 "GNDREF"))
  (pad "S1" thru_hole oval (at -4.32 -3.105 270) (size 1 2.1) (drill oval 0.6 1.7) (layers *.Cu *.Mask) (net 3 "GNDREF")))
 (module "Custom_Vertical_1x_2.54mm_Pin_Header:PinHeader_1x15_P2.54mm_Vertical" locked (layer "F.Cu") (at 14 44.48 90)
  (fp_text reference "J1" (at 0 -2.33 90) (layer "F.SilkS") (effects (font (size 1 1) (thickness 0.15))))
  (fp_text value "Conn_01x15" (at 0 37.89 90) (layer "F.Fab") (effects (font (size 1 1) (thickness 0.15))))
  (pad "15" thru_hole oval (at 0 35.56 90) (size 1.7 1.7) (drill 1) (layers *.Cu *.Mask) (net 3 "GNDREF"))
  (pad "14" thru_hole oval (at 0 33.02 90) (size 1.7 1.7) (drill 1) (layers *.Cu *.Mask) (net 6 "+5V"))
  (pad "13" thru_hole oval (at 0 30.48 90) (size 1.7 1.7) (drill 1) (layers *.Cu *.Mask) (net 10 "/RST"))
  (pad "12" thru_hole oval (at 0 27.94 90) (size 1.7 1.7) (drill 1) (layers *.Cu *.Mask) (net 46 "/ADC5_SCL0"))
  (pad "11" thru_hole oval (at 0 25.4 90) (size 1.7 1.7) (drill 1) (layers *.Cu *.Mask) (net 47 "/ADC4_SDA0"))
  (pad "10" thru_hole oval (at 0 22.86 90) (size 1.7 1.7) (drill 1) (layers *.Cu *.Mask) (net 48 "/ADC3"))
  (pad "9" thru_hole oval (at 0 20.32 90) (size 1.7 1.7) (drill 1) (layers *.Cu *.Mask) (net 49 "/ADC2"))
  (pad "8" thru_hole oval (at 0 17.78 90) (size 1.7 1.7) (drill 1) (layers *.Cu *.Mask) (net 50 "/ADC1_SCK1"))
  (pad "7" thru_hole oval (at 0 15.24 90) (size 1.7 1.7) (drill 1) (layers *.Cu *.Mask) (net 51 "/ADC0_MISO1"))
  (pad "6" thru_hole oval (at 0 12.7 90) (size 1.7 1.7) (drill 1) (layers *.Cu *.Mask) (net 21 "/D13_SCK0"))
  (pad "5" thru_hole oval (at 0 10.16 90) (size 1.7 1.7) (drill 1) (layers *.Cu *.Mask) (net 22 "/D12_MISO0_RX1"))
  (pad "4" thru_hole oval (at 0 7.62 90) (size 1.7 1.7) (drill 1) (layers *.Cu *.Mask) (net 20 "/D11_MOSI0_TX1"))
  (pad "3" thru_hole oval (at 0 5.08 90) (size 1.7 1.7) (drill 1) (layers *.Cu *.Mask) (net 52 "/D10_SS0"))
  (pad "2" thru_hole oval (at 0 2.54 90) (size 1.7 1.7) (drill 1) (layers *.Cu *.Mask) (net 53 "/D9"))
  (pad "1" thru_hole oval (at 0 0 90) (size 1.7 1.7) (drill 1) (layers *.Cu *.Mask) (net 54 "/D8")))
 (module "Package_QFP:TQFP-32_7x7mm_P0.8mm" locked (layer "F.Cu") (at 43 29)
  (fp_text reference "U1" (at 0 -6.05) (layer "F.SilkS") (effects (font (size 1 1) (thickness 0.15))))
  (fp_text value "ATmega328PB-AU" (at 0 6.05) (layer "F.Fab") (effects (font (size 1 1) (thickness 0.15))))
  (pad "32" smd rect (at -2.8 -4.25 90) (size 1.6 0.55) (layers "F.Cu" "F.Paste" "F.Mask") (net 43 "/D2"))
  (pad "31" smd rect (at -2 -4.25 90) (size 1.6 0.55) (layers "F.Cu" "F.Paste" "F.Mask") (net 18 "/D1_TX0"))
  (pad "30" smd rect (at -1.2 -4.25 90) (size 1.6 0.55) (layers "F.Cu" "F.Paste" "F.Mask") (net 17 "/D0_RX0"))
  (pad "29" smd rect (at -0.4 -4.25 90) (size 1.6 0.55) (layers "F.Cu" "F.Paste" "F.Mask") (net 10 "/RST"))
  (pad "28" smd rect (at 0.4 -4.25 90) (size 1.6 0.55) (layers "F.Cu" "F.Paste" "F.Mask") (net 46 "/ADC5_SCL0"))
  (pad "27" smd rect (at 1.2 -4.25 90) (size 1.6 0.55) (layers "F.Cu" "F.Paste" "F.Mask") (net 47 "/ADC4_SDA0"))
  (pad "26" smd rect (at 2 -4.25 90) (size 1.6 0.55) (layers "F.Cu" "F.Paste" "F.Mask") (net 48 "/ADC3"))
  (pad "25" smd rect (at 2.8 -4.25 90) (size 1.6 0.55) (layers "F.Cu" "F.Paste" "F.Mask") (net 49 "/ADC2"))
  (pad "24" smd rect (at 4.25 -2.8) (size 1.6 0.55) (layers "F.Cu" "F.Paste" "F.Mask") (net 50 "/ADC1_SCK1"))
  (pad "23" smd rect (at 4.25 -2) (size 1.6 0.55) (layers "F.Cu" "F.Paste" "F.Mask") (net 51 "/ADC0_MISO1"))
  (pad "22" smd rect (at 4.25 -1.2) (size 1.6 0.55) (layers "F.Cu" "F.Paste" "F.Mask") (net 34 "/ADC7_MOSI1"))
  (pad "21" smd rect (at 4.25 -0.4) (size 1.6 0.55) (layers "F.Cu" "F.Paste" "F.Mask") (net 3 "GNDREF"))
  (pad "20" smd rect (at 4.25 0.4) (size 1.6 0.55) (layers "F.Cu" "F.Paste" "F.Mask") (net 25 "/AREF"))
  (pad "19" smd rect (at 4.25 1.2) (size 1.6 0.55) (layers "F.Cu" "F.Paste" "F.Mask") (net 35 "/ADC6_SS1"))
  (pad "18" smd rect (at 4.25 2) (size 1.6 0.55) (layers "F.Cu" "F.Paste" "F.Mask") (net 6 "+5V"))
  (pad "17" smd rect (at 4.25 2.8) (size 1.6 0.55) (layers "F.Cu" "F.Paste" "F.Mask") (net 21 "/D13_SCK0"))
  (pad "16" smd rect (at 2.8 4.25 90) (size 1.6 0.55) (layers "F.Cu" "F.Paste" "F.Mask") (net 22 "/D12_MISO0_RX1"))
  (pad "15" smd rect (at 2 4.25 90) (size 1.6 0.55) (layers "F.Cu" "F.Paste" "F.Mask") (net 20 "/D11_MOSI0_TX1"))
  (pad "14" smd rect (at 1.2 4.25 90) (size 1.6 0.55) (layers "F.Cu" "F.Paste" "F.Mask") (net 52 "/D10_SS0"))
  (pad "13" smd rect (at 0.4 4.25 90) (size 1.6 0.55) (layers "F.Cu" "F.Paste" "F.Mask") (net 53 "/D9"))
  (pad "12" smd rect (at -0.4 4.25 90) (size 1.6 0.55) (layers "F.Cu" "F.Paste" "F.Mask") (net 54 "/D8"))
  (pad "11" smd rect (at -1.2 4.25 90) (size 1.6 0.55) (layers "F.Cu" "F.Paste" "F.Mask") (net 38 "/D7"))
  (pad "10" smd rect (at -2 4.25 90) (size 1.6 0.55) (layers "F.Cu" "F.Paste" "F.Mask") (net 39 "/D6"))
  (pad "9" smd rect (at -2.8 4.25 90) (size 1.6 0.55) (layers "F.Cu" "F.Paste" "F.Mask") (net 40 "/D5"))
  (pad "8" smd rect (at -4.25 2.8) (size 1.6 0.55) (layers "F.Cu" "F.Paste" "F.Mask") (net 13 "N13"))
  (pad "7" smd rect (at -4.25 2) (size 1.6 0.55) (layers "F.Cu" "F.Paste" "F.Mask") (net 14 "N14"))
  (pad "6" smd rect (at -4.25 1.2) (size 1.6 0.55) (layers "F.Cu" "F.Paste" "F.Mask") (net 36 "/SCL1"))
  (pad "5" smd rect (at -4.25 0.4) (size 1.6 0.55) (layers "F.Cu" "F.Paste" "F.Mask") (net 3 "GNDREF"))
  (pad "4" smd rect (at -4.25 -0.4) (size 1.6 0.55) (layers "F.Cu" "F.Paste" "F.Mask") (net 6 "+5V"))
  (pad "3" smd rect (at -4.25 -1.2) (size 1.6 0.55) (layers "F.Cu" "F.Paste" "F.Mask") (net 37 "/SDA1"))
  (pad "2" smd rect (at -4.25 -2) (size 1.6 0.55) (layers "F.Cu" "F.Paste" "F.Mask") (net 41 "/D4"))
  (pad "1" smd rect (at -4.25 -2.8) (size 1.6 0.55) (layers "F.Cu" "F.Paste" "F.Mask") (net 42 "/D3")))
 (gr_line (start 12 43) (end 12 12) (layer "Edge.Cuts") (width 0.05))
 (gr_line (start 12 46.48) (end 12 43) (layer "Edge.Cuts") (width 0.05))
 (gr_line (start 52 46.48) (end 12 46.48) (layer "Edge.Cuts") (width 0.05))
 (gr_line (start 52 12) (end 52 46.48) (layer "Edge.Cuts") (width 0.05))
 (gr_line (start 12 12) (end 52 12) (layer "Edge.Cuts") (width 0.05))
 (segment (start 19.557501 29.225) (end 18.695 29.225) (width 0.127) (layer "F.Cu") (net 32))
 (segment (start 18.695 29.225) (end 18.67 29.25) (width 0.127) (layer "F.Cu") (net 32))
 (segment (start 19.681065 29.761065) (end 19.7 29.78) (width 0.127) (layer "B.Cu") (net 32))
 (segment (start 19.681065 28.244373) (end 19.681065 29.761065) (width 0.127) (layer "B.Cu") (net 32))
 (via (at 19.681065 28.244373) (size 0.6) (drill 0.35) (layers "F.Cu" "B.Cu") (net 32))
 (via (at 19.7 29.78) (size 0.6) (drill 0.35) (layers "F.Cu" "B.Cu") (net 32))
 (segment (start 19.661129 28.25) (end 19.675438 28.25) (width 0.127) (layer "F.Cu") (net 32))
 (segment (start 19.7 29.78) (end 19.557501 29.637501) (width 0.127) (layer "F.Cu") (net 32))
 (segment (start 19.675438 28.25) (end 19.681065 28.244373) (width 0.127) (layer "F.Cu") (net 32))
 (segment (start 19.557501 29.637501) (end 19.557501 29.225) (width 0.127) (layer "F.Cu") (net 32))
 (segment (start 21.62 14) (end 28.98 21.36) (width 0.127) (layer "F.Cu") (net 42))
 (segment (start 28.98 21.36) (end 30.91 21.36) (width 0.127) (layer "F.Cu") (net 42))
 (segment (start 36.65 35.89) (end 36.65 35.332902) (width 0.127) (layer "F.Cu") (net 14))
 (segment (start 38.132098 31) (end 38.75 31) (width 0.127) (layer "F.Cu") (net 14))
 (segment (start 36.65 35.332902) (end 37.559499 34.423403) (width 0.127) (layer "F.Cu") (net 14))
 (segment (start 37.559499 34.423403) (end 37.559499 31.572599) (width 0.127) (layer "F.Cu") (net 14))
 (segment (start 37.559499 31.572599) (end 38.132098 31) (width 0.127) (layer "F.Cu") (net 14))
 (segment (start 38.35 33.69) (end 38.35 32.2) (width 0.127) (layer "F.Cu") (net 13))
 (segment (start 38.35 32.2) (end 38.75 31.8) (width 0.127) (layer "F.Cu") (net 13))
 (segment (start 25.525 33.445) (end 25.136499 33.833501) (width 0.127) (layer "F.Cu") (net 11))
 (segment (start 25.136499 36.336499) (end 26 37.2) (width 0.127) (layer "F.Cu") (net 11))
 (segment (start 25.136499 33.833501) (end 25.136499 36.336499) (width 0.127) (layer "F.Cu") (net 11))
 (segment (start 25.525 32.175) (end 26.5 32.175) (width 0.127) (layer "F.Cu") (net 12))
 (segment (start 26.5 32.175) (end 27.7 33.375) (width 0.127) (layer "F.Cu") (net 12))
 (segment (start 27.7 33.375) (end 27.7 35) (width 0.127) (layer "F.Cu") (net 12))
 (segment (start 17.639489 15.099489) (end 17.639489 19.49756) (width 0.127) (layer "F.Cu") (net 18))
 (segment (start 16.54 14) (end 17.639489 15.099489) (width 0.127) (layer "F.Cu") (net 18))
 (segment (start 17.639489 19.49756) (end 25.23693 27.095) (width 0.127) (layer "F.Cu") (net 18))
 (segment (start 25.23693 27.095) (end 25.525 27.095) (width 0.127) (layer "F.Cu") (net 18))
 (segment (start 15.113501 12.886499) (end 17.074481 12.886499) (width 0.127) (layer "F.Cu") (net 17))
 (segment (start 14 14) (end 15.113501 12.886499) (width 0.127) (layer "F.Cu") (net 17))
 (segment (start 17.074481 12.886499) (end 17.966499 13.778517) (width 0.127) (layer "F.Cu") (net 17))
 (segment (start 17.966499 13.778517) (end 17.966499 19.362109) (width 0.127) (layer "F.Cu") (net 17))
 (segment (start 17.966499 19.362109) (end 24.42939 25.825) (width 0.127) (layer "F.Cu") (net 17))
 (segment (start 24.42939 25.825) (end 25.525 25.825) (width 0.127) (layer "F.Cu") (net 17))
 (segment (start 25.525 27.095) (end 26.37693 27.095) (width 0.127) (layer "F.Cu") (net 18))
 (segment (start 18.67 28.75) (end 17.968 28.75) (width 0.127) (layer "F.Cu") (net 33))
 (segment (start 17.968 28.75) (end 17.831499 28.886501) (width 0.127) (layer "F.Cu") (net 33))
 (segment (start 17.831499 29.610801) (end 17.970698 29.75) (width 0.127) (layer "F.Cu") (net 33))
 (segment (start 17.970698 29.75) (end 18.67 29.75) (width 0.127) (layer "F.Cu") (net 33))
 (segment (start 17.831499 28.886501) (end 17.831499 29.610801) (width 0.127) (layer "F.Cu") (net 33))
 (segment (start 18.67 28.25) (end 19.661129 28.25) (width 0.127) (layer "F.Cu") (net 32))
 (segment (start 24.85501 30.23501) (end 25.525 30.905) (width 0.2) (layer "F.Cu") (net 32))
 (segment (start 24.51532 30.23501) (end 24.85501 30.23501) (width 0.2) (layer "F.Cu") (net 32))
 (segment (start 24.031397 28.775) (end 24.891397 29.635) (width 0.2) (layer "F.Cu") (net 33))
 (segment (start 19.557501 28.775) (end 24.031397 28.775) (width 0.2) (layer "F.Cu") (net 33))
 (segment (start 19.557501 29.225) (end 23.845 29.225) (width 0.2) (layer "F.Cu") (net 32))
 (segment (start 24.891397 29.635) (end 25.525 29.635) (width 0.2) (layer "F.Cu") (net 33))
 (segment (start 24.24999 29.62999) (end 24.24999 29.96968) (width 0.2) (layer "F.Cu") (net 32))
 (segment (start 19.532501 28.75) (end 19.557501 28.775) (width 0.2) (layer "F.Cu") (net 33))
 (segment (start 18.67 28.75) (end 19.532501 28.75) (width 0.2) (layer "F.Cu") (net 33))
 (segment (start 24.24999 29.96968) (end 24.51532 30.23501) (width 0.2) (layer "F.Cu") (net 32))
 (segment (start 23.845 29.225) (end 24.24999 29.62999) (width 0.2) (layer "F.Cu") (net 32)))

